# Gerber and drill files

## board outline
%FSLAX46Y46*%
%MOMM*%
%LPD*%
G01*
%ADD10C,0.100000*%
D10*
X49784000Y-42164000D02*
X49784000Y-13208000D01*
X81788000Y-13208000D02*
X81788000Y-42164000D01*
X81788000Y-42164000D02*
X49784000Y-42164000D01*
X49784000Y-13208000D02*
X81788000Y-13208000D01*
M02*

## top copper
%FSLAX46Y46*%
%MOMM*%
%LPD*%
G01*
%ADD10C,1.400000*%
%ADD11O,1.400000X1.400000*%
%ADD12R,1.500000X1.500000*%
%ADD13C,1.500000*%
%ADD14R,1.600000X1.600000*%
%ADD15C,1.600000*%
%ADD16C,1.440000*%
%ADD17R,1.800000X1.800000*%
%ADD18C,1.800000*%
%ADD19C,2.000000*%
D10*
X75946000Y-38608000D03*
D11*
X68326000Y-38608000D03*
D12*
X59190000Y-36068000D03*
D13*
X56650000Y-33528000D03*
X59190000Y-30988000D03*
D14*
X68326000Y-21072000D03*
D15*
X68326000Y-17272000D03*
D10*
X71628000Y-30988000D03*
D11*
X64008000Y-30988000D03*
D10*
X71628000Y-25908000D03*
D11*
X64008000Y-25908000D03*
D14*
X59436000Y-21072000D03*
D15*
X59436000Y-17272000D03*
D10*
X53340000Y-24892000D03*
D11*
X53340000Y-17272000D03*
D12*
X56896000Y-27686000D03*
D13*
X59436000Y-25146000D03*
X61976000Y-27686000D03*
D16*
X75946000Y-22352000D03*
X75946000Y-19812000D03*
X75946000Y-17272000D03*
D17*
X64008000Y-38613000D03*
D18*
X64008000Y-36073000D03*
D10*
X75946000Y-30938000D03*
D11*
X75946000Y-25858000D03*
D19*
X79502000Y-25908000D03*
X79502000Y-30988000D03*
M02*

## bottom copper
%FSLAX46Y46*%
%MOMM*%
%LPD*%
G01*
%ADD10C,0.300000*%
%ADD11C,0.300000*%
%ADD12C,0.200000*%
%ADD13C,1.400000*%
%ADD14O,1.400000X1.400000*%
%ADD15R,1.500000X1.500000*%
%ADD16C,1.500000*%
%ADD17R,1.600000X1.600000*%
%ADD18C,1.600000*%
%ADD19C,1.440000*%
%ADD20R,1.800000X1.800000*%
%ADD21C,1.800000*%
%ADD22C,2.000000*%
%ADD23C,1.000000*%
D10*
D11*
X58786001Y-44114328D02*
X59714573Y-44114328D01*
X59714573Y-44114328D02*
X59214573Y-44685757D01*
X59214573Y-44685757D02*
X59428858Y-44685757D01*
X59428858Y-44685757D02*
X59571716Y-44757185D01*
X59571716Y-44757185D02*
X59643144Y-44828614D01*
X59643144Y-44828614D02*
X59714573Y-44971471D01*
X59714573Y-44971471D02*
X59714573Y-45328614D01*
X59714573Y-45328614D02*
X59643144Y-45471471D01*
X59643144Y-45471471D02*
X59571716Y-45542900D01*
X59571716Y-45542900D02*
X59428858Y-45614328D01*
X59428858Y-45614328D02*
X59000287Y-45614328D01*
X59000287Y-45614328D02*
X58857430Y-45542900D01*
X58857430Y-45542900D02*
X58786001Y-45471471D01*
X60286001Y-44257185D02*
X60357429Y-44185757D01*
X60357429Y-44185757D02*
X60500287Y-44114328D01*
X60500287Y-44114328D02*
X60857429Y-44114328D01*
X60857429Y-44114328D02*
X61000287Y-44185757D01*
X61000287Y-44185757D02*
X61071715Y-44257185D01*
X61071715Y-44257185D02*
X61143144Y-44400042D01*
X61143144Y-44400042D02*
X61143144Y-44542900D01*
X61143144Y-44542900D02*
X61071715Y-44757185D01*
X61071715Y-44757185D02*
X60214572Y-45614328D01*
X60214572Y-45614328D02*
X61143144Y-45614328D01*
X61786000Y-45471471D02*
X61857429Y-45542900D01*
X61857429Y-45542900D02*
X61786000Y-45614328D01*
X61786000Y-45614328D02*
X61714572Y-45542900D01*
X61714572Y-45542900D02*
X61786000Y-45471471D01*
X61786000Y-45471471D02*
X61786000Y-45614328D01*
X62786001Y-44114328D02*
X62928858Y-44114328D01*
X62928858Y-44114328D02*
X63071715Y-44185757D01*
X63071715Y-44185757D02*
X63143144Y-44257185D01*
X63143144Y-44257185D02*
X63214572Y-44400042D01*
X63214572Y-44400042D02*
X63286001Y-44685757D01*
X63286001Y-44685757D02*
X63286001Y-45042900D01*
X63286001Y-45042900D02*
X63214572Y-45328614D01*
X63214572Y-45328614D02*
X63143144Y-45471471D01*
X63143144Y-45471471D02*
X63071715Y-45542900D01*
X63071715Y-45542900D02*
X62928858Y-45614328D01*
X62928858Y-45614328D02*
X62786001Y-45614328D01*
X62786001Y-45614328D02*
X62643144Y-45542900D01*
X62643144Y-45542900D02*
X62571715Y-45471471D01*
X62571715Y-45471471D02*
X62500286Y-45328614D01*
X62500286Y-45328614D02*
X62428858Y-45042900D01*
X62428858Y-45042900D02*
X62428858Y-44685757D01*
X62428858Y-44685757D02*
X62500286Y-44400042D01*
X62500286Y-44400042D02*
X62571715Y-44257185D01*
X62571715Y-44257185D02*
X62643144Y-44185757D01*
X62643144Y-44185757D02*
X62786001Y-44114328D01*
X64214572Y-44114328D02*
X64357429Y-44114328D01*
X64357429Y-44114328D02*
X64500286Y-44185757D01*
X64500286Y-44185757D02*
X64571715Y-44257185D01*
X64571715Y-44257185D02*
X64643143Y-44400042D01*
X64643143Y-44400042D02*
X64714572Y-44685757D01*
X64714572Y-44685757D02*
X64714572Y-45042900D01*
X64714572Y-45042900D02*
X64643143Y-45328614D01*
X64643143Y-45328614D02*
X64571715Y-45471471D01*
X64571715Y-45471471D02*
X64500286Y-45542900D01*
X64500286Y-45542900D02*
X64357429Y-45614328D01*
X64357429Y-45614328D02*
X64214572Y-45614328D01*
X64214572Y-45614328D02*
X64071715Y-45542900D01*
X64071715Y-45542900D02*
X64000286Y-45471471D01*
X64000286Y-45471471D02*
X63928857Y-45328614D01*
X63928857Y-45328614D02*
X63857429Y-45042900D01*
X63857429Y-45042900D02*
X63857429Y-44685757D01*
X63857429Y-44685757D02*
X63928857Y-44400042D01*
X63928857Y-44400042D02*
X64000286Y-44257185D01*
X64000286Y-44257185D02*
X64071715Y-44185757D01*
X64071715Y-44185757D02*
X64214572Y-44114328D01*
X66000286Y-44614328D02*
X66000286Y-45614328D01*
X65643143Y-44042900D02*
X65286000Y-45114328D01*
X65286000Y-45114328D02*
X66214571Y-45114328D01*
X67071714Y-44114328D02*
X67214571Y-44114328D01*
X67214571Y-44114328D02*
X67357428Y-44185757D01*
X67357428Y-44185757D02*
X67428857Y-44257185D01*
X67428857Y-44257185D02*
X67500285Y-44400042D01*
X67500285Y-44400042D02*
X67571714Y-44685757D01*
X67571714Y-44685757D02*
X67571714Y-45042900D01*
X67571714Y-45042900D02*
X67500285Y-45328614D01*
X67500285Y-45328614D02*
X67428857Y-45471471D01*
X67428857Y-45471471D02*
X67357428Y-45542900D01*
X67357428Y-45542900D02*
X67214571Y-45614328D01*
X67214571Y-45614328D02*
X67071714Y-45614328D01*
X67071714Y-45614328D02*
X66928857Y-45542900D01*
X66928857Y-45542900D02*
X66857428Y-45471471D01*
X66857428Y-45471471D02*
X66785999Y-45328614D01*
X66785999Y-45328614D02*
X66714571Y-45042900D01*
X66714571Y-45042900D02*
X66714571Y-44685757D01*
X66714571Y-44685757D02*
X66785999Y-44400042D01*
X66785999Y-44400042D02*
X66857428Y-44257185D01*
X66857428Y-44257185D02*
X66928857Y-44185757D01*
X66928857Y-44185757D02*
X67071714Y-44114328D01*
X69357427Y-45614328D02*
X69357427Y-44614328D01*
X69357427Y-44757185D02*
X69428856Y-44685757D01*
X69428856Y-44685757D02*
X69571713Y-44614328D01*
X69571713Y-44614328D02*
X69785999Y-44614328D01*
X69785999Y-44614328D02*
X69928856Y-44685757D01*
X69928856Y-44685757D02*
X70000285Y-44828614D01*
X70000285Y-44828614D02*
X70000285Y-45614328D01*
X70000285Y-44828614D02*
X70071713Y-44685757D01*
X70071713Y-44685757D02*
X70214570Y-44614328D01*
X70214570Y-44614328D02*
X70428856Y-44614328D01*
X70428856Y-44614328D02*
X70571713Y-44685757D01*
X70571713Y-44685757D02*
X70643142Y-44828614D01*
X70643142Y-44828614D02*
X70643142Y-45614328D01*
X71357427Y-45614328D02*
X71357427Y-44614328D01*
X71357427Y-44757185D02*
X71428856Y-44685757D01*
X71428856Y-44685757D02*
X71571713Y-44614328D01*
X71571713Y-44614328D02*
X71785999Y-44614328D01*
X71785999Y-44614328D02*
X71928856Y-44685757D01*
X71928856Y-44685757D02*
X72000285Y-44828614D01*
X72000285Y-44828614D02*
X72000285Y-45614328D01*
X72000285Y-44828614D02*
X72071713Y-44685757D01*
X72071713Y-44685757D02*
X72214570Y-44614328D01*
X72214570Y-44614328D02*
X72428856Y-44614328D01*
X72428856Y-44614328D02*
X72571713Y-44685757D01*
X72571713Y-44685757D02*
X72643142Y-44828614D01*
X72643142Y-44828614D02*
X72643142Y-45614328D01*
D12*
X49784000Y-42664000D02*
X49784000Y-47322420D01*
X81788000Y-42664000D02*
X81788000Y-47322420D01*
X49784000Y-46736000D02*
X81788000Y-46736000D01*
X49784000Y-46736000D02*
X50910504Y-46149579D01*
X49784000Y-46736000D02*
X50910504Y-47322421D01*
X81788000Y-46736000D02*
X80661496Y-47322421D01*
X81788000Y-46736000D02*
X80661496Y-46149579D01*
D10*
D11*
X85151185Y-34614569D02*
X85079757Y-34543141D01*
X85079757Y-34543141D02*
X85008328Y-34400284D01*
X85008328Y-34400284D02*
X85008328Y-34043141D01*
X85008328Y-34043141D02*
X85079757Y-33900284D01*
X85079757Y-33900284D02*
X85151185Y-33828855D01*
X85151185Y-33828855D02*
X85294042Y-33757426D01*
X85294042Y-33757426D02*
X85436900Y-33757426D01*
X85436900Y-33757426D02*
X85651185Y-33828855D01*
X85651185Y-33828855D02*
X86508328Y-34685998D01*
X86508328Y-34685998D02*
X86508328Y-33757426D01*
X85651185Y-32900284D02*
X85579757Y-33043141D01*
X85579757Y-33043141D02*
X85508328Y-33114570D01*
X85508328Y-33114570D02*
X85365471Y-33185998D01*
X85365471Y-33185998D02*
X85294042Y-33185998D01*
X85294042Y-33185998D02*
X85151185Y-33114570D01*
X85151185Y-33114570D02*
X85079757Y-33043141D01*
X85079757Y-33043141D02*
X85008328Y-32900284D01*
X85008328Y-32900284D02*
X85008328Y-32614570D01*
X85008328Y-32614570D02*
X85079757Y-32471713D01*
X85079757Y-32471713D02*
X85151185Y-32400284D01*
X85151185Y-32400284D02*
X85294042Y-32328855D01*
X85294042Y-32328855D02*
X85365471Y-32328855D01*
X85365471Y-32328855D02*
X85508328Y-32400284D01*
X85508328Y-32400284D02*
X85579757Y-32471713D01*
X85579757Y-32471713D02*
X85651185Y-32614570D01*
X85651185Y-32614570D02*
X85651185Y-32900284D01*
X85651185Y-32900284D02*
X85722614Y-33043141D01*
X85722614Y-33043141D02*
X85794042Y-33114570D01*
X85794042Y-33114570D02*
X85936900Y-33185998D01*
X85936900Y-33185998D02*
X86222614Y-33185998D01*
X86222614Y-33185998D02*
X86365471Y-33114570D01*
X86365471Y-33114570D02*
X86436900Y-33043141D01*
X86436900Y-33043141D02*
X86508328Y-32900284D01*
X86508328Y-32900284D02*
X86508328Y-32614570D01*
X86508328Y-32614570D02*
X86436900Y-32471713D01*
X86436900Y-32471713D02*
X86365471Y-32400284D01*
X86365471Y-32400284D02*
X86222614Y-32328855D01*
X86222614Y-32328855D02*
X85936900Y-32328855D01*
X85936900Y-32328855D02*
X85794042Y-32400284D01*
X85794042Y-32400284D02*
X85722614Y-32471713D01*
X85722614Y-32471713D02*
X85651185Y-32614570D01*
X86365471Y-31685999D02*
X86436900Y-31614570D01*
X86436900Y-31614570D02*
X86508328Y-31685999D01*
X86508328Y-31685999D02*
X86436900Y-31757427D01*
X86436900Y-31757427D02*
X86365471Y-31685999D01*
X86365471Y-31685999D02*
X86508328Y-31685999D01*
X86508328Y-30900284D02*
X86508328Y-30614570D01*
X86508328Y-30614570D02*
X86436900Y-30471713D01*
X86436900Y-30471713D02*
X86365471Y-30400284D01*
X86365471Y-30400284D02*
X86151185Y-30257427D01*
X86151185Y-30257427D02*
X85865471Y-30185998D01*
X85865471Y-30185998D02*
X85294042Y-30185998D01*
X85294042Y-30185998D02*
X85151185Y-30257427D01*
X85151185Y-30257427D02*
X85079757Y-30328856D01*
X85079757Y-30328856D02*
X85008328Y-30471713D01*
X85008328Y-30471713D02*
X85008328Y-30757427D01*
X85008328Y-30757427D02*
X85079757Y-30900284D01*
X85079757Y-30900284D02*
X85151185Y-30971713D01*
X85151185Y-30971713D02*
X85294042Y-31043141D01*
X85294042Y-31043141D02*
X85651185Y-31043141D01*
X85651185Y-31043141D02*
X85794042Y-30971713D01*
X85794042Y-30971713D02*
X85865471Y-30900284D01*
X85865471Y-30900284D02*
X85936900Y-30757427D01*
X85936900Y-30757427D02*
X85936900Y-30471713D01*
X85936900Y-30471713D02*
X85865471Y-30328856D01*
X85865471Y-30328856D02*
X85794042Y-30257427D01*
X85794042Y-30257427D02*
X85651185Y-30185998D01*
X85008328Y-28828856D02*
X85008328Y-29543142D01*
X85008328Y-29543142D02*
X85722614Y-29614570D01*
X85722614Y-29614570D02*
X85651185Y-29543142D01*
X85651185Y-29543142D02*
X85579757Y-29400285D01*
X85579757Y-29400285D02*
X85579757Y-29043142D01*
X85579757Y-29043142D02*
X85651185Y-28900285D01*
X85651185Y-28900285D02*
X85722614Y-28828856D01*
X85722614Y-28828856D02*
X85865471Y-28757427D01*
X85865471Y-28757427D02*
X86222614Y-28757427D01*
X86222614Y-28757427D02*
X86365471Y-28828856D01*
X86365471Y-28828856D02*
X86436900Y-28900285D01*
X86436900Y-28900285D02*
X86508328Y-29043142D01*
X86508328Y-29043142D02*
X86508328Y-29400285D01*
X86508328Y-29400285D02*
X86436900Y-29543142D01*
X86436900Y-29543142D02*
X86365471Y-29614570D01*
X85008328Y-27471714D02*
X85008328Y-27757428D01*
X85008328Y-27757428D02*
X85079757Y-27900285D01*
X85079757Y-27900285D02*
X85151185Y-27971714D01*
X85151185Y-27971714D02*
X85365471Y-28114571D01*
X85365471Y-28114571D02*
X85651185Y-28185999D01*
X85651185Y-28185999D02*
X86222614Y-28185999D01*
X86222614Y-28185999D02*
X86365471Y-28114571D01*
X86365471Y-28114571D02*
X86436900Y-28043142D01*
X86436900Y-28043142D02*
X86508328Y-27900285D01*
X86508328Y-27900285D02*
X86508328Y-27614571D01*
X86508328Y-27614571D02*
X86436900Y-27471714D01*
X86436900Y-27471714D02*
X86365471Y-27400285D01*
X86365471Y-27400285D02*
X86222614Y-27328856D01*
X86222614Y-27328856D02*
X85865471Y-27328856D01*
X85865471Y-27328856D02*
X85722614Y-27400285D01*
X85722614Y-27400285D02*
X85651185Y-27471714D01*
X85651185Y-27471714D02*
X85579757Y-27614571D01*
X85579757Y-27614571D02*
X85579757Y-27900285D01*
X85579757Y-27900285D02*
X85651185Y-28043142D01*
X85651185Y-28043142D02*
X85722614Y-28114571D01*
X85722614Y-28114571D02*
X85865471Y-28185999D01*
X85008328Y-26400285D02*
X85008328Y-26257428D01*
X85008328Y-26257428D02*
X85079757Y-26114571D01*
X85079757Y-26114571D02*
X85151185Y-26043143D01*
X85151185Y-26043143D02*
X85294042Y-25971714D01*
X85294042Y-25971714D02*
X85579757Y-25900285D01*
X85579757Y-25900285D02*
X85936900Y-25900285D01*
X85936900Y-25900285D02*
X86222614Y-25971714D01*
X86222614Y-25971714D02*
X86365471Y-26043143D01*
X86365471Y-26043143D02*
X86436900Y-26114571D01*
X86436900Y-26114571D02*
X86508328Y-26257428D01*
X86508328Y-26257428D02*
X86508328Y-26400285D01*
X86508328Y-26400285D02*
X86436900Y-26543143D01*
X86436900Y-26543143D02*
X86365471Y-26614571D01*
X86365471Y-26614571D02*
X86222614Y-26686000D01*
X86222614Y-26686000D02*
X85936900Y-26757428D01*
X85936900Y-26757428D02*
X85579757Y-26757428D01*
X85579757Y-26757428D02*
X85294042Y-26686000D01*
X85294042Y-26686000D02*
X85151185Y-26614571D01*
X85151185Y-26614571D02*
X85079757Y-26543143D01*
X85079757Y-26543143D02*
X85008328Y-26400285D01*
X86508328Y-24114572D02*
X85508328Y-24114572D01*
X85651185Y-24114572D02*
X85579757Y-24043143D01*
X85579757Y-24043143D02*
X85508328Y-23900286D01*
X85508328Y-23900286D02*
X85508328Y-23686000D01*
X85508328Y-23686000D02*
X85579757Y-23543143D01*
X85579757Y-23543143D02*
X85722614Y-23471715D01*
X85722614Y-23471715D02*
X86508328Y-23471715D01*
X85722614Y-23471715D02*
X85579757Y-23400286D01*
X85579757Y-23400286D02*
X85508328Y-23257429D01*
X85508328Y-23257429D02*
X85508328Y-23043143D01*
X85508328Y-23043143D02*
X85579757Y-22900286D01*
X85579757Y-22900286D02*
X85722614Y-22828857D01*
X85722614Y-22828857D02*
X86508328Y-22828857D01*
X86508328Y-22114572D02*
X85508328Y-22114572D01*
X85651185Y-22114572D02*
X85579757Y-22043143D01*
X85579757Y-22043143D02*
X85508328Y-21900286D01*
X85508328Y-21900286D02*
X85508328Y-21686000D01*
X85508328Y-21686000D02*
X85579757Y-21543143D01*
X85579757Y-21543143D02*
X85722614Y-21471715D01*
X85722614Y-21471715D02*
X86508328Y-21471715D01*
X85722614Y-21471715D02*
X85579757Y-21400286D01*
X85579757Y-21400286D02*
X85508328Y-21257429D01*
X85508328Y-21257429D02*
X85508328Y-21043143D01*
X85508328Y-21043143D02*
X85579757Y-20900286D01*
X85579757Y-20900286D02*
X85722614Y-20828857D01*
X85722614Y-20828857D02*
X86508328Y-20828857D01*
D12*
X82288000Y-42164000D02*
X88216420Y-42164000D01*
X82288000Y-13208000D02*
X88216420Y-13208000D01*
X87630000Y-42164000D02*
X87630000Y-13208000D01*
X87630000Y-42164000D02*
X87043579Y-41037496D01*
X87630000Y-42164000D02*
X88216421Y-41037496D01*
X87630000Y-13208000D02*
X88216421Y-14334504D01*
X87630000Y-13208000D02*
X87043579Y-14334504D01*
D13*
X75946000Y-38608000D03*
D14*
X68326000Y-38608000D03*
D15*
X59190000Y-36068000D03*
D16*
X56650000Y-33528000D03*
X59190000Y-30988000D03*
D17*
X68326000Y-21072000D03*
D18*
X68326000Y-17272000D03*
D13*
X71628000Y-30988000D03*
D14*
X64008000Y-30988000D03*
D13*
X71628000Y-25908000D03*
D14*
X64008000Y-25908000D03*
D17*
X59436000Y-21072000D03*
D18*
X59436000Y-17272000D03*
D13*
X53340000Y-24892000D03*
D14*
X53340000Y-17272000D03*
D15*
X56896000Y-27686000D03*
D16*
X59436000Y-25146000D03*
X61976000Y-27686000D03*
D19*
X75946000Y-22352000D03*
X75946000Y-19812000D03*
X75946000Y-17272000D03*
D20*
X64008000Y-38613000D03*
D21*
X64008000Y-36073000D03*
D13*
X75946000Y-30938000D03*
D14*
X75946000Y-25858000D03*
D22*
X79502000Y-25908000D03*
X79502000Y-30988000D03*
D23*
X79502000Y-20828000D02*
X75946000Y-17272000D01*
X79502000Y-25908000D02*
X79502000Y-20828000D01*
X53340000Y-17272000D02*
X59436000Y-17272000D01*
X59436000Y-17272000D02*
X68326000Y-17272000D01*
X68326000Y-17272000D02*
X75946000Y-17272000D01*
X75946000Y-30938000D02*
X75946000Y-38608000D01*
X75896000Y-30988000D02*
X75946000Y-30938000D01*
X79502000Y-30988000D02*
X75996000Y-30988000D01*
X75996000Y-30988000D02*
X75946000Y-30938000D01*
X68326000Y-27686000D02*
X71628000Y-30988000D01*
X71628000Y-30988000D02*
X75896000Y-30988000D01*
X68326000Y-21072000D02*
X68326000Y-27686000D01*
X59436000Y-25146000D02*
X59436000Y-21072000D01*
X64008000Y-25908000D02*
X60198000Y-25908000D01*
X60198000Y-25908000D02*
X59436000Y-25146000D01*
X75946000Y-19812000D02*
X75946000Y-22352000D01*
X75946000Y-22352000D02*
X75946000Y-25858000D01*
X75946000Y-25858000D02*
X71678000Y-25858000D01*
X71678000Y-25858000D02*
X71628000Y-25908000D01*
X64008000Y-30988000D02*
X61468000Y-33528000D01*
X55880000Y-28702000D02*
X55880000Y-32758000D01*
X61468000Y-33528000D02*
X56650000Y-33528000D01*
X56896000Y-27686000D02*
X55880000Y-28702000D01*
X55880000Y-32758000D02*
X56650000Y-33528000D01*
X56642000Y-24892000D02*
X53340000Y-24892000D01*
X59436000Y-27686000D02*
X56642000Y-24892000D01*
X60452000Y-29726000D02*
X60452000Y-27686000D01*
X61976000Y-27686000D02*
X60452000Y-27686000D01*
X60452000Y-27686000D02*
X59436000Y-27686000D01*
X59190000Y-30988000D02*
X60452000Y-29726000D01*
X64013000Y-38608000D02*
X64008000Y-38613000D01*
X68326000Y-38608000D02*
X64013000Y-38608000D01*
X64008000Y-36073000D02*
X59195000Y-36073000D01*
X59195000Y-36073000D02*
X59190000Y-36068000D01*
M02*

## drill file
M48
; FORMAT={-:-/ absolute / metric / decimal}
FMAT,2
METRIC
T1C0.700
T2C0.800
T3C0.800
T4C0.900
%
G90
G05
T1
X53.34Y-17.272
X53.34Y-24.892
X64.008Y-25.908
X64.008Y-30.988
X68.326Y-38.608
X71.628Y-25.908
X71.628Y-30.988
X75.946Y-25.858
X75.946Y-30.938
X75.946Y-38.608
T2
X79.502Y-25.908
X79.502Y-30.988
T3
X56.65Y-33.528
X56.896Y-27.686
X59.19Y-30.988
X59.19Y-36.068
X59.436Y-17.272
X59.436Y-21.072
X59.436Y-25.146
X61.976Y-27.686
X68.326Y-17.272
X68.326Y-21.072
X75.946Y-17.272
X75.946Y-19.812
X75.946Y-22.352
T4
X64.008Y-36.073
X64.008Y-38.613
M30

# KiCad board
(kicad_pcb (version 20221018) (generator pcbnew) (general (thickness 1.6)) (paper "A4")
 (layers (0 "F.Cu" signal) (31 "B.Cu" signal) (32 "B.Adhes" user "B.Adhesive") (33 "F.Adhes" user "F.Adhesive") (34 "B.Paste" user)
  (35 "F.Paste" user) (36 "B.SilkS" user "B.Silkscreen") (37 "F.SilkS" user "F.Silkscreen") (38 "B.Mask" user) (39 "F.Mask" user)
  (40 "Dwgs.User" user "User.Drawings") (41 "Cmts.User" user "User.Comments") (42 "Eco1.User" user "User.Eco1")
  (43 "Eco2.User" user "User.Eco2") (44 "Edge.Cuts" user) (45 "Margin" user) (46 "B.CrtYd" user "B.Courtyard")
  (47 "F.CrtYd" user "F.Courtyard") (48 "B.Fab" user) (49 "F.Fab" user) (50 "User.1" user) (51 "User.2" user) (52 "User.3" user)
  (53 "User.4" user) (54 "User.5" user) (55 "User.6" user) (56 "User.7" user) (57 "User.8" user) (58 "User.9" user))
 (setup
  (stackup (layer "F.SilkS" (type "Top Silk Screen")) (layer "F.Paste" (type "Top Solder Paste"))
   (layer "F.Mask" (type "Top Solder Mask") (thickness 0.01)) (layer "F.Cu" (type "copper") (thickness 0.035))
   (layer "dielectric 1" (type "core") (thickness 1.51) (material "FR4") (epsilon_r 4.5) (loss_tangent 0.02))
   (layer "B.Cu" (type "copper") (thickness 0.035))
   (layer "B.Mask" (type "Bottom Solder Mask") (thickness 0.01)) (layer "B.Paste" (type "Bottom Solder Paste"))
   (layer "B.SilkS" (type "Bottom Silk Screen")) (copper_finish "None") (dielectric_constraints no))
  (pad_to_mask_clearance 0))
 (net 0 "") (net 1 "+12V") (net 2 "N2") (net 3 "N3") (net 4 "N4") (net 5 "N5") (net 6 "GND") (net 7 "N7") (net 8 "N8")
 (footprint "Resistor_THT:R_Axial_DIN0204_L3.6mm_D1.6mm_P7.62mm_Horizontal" (layer "F.Cu") (at 75.946 38.608 180)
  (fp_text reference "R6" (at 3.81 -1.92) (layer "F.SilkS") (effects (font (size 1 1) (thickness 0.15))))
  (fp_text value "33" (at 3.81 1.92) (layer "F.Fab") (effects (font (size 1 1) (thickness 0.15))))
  (pad "1" thru_hole circle (at 0 0 180) (size 1.4 1.4) (drill 0.7) (layers "*.Cu" "*.Mask") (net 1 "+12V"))
  (pad "2" thru_hole oval (at 7.62 0 180) (size 1.4 1.4) (drill 0.7) (layers "*.Cu" "*.Mask") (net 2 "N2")))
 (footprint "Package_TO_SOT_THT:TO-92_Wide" (layer "F.Cu") (at 59.19 36.068 90)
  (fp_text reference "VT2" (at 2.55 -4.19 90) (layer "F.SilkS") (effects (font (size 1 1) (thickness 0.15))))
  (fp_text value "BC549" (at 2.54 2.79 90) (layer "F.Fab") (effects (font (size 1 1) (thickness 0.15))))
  (pad "1" thru_hole rect (at 0 0 90) (size 1.5 1.5) (drill 0.8) (layers "*.Cu" "*.Mask") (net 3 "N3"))
  (pad "2" thru_hole circle (at 2.54 -2.54 90) (size 1.5 1.5) (drill 0.8) (layers "*.Cu" "*.Mask") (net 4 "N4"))
  (pad "3" thru_hole circle (at 5.08 0 90) (size 1.5 1.5) (drill 0.8) (layers "*.Cu" "*.Mask") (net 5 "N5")))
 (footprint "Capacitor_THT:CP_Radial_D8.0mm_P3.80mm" (layer "F.Cu") (at 68.326 21.072 90)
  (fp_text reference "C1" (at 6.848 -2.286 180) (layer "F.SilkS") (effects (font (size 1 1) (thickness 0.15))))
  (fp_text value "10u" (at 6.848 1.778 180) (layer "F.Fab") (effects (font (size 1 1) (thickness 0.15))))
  (pad "1" thru_hole rect (at 0 0 90) (size 1.6 1.6) (drill 0.8) (layers "*.Cu" "*.Mask") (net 1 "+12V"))
  (pad "2" thru_hole circle (at 3.8 0 90) (size 1.6 1.6) (drill 0.8) (layers "*.Cu" "*.Mask") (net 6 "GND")))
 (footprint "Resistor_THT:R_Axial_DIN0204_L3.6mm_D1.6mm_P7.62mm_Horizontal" (layer "F.Cu") (at 71.628 30.988 180)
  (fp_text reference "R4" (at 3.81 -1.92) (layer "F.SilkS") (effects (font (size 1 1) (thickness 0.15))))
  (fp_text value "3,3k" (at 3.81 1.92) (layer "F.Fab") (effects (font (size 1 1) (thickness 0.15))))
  (pad "1" thru_hole circle (at 0 0 180) (size 1.4 1.4) (drill 0.7) (layers "*.Cu" "*.Mask") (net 1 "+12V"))
  (pad "2" thru_hole oval (at 7.62 0 180) (size 1.4 1.4) (drill 0.7) (layers "*.Cu" "*.Mask") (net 4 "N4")))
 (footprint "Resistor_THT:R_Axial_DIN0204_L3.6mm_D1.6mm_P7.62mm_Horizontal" (layer "F.Cu") (at 71.628 25.908 180)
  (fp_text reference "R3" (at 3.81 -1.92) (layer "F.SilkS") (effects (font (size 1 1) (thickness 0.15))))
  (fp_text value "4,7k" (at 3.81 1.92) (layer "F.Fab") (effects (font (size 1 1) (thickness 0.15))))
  (pad "1" thru_hole circle (at 0 0 180) (size 1.4 1.4) (drill 0.7) (layers "*.Cu" "*.Mask") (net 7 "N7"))
  (pad "2" thru_hole oval (at 7.62 0 180) (size 1.4 1.4) (drill 0.7) (layers "*.Cu" "*.Mask") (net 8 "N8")))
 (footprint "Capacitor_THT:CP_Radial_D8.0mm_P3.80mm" (layer "F.Cu") (at 59.436 21.072 90)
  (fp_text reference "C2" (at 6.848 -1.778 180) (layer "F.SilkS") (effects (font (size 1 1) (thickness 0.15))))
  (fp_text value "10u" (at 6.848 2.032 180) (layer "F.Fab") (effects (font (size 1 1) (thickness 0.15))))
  (pad "1" thru_hole rect (at 0 0 90) (size 1.6 1.6) (drill 0.8) (layers "*.Cu" "*.Mask") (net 8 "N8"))
  (pad "2" thru_hole circle (at 3.8 0 90) (size 1.6 1.6) (drill 0.8) (layers "*.Cu" "*.Mask") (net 6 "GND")))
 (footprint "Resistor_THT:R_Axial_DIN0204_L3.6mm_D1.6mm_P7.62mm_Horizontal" (layer "F.Cu") (at 53.34 24.892 90)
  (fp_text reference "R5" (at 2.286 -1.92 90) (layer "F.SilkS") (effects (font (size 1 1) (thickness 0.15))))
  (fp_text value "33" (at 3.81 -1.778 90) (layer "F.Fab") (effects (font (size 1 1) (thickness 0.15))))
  (pad "1" thru_hole circle (at 0 0 90) (size 1.4 1.4) (drill 0.7) (layers "*.Cu" "*.Mask") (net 5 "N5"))
  (pad "2" thru_hole oval (at 7.62 0 90) (size 1.4 1.4) (drill 0.7) (layers "*.Cu" "*.Mask") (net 6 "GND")))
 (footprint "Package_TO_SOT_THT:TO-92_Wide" (layer "F.Cu") (at 56.896 27.686)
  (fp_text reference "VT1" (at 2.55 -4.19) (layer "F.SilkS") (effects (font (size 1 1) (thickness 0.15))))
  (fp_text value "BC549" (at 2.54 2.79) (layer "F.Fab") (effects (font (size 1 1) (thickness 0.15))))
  (pad "1" thru_hole rect (at 0 0) (size 1.5 1.5) (drill 0.8) (layers "*.Cu" "*.Mask") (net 4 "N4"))
  (pad "2" thru_hole circle (at 2.54 -2.54) (size 1.5 1.5) (drill 0.8) (layers "*.Cu" "*.Mask") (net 8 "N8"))
  (pad "3" thru_hole circle (at 5.08 0) (size 1.5 1.5) (drill 0.8) (layers "*.Cu" "*.Mask") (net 5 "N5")))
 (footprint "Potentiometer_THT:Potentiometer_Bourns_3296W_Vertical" (layer "F.Cu") (at 75.946 22.352 -90)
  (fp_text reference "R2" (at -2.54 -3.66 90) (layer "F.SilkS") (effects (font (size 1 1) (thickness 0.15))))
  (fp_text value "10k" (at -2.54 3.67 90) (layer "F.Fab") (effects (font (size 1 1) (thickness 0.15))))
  (pad "1" thru_hole circle (at 0 0 270) (size 1.44 1.44) (drill 0.8) (layers "*.Cu" "*.Mask") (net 7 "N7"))
  (pad "2" thru_hole circle (at -2.54 0 270) (size 1.44 1.44) (drill 0.8) (layers "*.Cu" "*.Mask") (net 7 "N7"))
  (pad "3" thru_hole circle (at -5.08 0 270) (size 1.44 1.44) (drill 0.8) (layers "*.Cu" "*.Mask") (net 6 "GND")))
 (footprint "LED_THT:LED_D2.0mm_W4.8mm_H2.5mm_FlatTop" (layer "F.Cu") (at 64.008 38.613 90)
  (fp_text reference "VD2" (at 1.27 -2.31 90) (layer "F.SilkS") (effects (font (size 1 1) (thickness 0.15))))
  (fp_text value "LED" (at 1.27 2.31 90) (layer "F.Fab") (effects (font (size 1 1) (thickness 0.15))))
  (pad "1" thru_hole rect (at 0 0 90) (size 1.8 1.8) (drill 0.9) (layers "*.Cu" "*.Mask") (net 2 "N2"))
  (pad "2" thru_hole circle (at 2.54 0 90) (size 1.8 1.8) (drill 0.9) (layers "*.Cu" "*.Mask") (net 3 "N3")))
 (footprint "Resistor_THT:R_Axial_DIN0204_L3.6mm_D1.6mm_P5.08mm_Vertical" (layer "F.Cu") (at 75.946 30.938 90)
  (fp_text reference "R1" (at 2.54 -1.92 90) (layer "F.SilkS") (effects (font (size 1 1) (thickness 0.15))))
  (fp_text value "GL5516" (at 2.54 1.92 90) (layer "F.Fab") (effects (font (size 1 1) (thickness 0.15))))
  (pad "1" thru_hole circle (at 0 0 90) (size 1.4 1.4) (drill 0.7) (layers "*.Cu" "*.Mask") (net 1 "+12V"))
  (pad "2" thru_hole oval (at 5.08 0 90) (size 1.4 1.4) (drill 0.7) (layers "*.Cu" "*.Mask") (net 7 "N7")))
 (gr_line (start 49.784 42.164) (end 49.784 13.208) (stroke (width 0.1) (type default)) (layer "Edge.Cuts"))
 (gr_line (start 81.788 13.208) (end 81.788 42.164) (stroke (width 0.1) (type default)) (layer "Edge.Cuts"))
 (gr_line (start 81.788 42.164) (end 49.784 42.164) (stroke (width 0.1) (type default)) (layer "Edge.Cuts"))
 (gr_line (start 49.784 13.208) (end 81.788 13.208) (stroke (width 0.1) (type default)) (layer "Edge.Cuts"))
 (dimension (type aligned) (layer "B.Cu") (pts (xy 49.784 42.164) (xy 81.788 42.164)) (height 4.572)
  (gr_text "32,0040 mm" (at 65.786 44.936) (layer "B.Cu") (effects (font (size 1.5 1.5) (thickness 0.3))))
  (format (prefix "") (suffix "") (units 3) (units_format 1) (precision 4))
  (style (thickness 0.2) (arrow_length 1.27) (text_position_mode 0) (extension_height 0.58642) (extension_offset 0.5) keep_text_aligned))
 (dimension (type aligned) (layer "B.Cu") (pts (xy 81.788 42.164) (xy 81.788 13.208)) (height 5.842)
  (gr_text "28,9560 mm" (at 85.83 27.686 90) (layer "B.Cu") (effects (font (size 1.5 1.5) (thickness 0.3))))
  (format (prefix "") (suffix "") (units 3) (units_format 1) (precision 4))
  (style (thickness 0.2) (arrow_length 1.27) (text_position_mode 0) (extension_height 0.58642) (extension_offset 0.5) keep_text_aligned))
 (via blind (at 79.502 25.908) (size 2) (drill 0.8) (layers "F.Cu" "B.Cu") (free) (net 6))
 (segment (start 79.502 20.828) (end 75.946 17.272) (width 1) (layer "B.Cu") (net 6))
 (segment (start 79.502 25.908) (end 79.502 20.828) (width 1) (layer "B.Cu") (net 6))
 (segment (start 53.34 17.272) (end 59.436 17.272) (width 1) (layer "B.Cu") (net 6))
 (segment (start 59.436 17.272) (end 68.326 17.272) (width 1) (layer "B.Cu") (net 6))
 (segment (start 68.326 17.272) (end 75.946 17.272) (width 1) (layer "B.Cu") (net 6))
 (via blind (at 79.502 30.988) (size 2) (drill 0.8) (layers "F.Cu" "B.Cu") (free) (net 1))
 (segment (start 75.946 30.938) (end 75.946 38.608) (width 1) (layer "B.Cu") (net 1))
 (segment (start 75.896 30.988) (end 75.946 30.938) (width 1) (layer "B.Cu") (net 1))
 (segment (start 79.502 30.988) (end 75.996 30.988) (width 1) (layer "B.Cu") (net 1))
 (segment (start 75.996 30.988) (end 75.946 30.938) (width 1) (layer "B.Cu") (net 1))
 (segment (start 68.326 27.686) (end 71.628 30.988) (width 1) (layer "B.Cu") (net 1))
 (segment (start 71.628 30.988) (end 75.896 30.988) (width 1) (layer "B.Cu") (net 1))
 (segment (start 68.326 21.072) (end 68.326 27.686) (width 1) (layer "B.Cu") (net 1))
 (segment (start 59.436 25.146) (end 59.436 21.072) (width 1) (layer "B.Cu") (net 8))
 (segment (start 64.008 25.908) (end 60.198 25.908) (width 1) (layer "B.Cu") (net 8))
 (segment (start 60.198 25.908) (end 59.436 25.146) (width 1) (layer "B.Cu") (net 8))
 (segment (start 75.946 19.812) (end 75.946 22.352) (width 1) (layer "B.Cu") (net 7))
 (segment (start 75.946 22.352) (end 75.946 25.858) (width 1) (layer "B.Cu") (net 7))
 (segment (start 75.946 25.858) (end 71.678 25.858) (width 1) (layer "B.Cu") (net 7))
 (segment (start 71.678 25.858) (end 71.628 25.908) (width 1) (layer "B.Cu") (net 7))
 (segment (start 64.008 30.988) (end 61.468 33.528) (width 1) (layer "B.Cu") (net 4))
 (segment (start 55.88 28.702) (end 55.88 32.758) (width 1) (layer "B.Cu") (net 4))
 (segment (start 61.468 33.528) (end 56.65 33.528) (width 1) (layer "B.Cu") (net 4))
 (segment (start 56.896 27.686) (end 55.88 28.702) (width 1) (layer "B.Cu") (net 4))
 (segment (start 55.88 32.758) (end 56.65 33.528) (width 1) (layer "B.Cu") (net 4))
 (segment (start 56.642 24.892) (end 53.34 24.892) (width 1) (layer "B.Cu") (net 5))
 (segment (start 59.436 27.686) (end 56.642 24.892) (width 1) (layer "B.Cu") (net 5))
 (segment (start 60.452 29.726) (end 60.452 27.686) (width 1) (layer "B.Cu") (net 5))
 (segment (start 61.976 27.686) (end 60.452 27.686) (width 1) (layer "B.Cu") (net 5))
 (segment (start 60.452 27.686) (end 59.436 27.686) (width 1) (layer "B.Cu") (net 5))
 (segment (start 59.19 30.988) (end 60.452 29.726) (width 1) (layer "B.Cu") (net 5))
 (segment (start 64.013 38.608) (end 64.008 38.613) (width 1) (layer "B.Cu") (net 2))
 (segment (start 68.326 38.608) (end 64.013 38.608) (width 1) (layer "B.Cu") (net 2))
 (segment (start 64.008 36.073) (end 59.195 36.073) (width 1) (layer "B.Cu") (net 3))
 (segment (start 59.195 36.073) (end 59.19 36.068) (width 1) (layer "B.Cu") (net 3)))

